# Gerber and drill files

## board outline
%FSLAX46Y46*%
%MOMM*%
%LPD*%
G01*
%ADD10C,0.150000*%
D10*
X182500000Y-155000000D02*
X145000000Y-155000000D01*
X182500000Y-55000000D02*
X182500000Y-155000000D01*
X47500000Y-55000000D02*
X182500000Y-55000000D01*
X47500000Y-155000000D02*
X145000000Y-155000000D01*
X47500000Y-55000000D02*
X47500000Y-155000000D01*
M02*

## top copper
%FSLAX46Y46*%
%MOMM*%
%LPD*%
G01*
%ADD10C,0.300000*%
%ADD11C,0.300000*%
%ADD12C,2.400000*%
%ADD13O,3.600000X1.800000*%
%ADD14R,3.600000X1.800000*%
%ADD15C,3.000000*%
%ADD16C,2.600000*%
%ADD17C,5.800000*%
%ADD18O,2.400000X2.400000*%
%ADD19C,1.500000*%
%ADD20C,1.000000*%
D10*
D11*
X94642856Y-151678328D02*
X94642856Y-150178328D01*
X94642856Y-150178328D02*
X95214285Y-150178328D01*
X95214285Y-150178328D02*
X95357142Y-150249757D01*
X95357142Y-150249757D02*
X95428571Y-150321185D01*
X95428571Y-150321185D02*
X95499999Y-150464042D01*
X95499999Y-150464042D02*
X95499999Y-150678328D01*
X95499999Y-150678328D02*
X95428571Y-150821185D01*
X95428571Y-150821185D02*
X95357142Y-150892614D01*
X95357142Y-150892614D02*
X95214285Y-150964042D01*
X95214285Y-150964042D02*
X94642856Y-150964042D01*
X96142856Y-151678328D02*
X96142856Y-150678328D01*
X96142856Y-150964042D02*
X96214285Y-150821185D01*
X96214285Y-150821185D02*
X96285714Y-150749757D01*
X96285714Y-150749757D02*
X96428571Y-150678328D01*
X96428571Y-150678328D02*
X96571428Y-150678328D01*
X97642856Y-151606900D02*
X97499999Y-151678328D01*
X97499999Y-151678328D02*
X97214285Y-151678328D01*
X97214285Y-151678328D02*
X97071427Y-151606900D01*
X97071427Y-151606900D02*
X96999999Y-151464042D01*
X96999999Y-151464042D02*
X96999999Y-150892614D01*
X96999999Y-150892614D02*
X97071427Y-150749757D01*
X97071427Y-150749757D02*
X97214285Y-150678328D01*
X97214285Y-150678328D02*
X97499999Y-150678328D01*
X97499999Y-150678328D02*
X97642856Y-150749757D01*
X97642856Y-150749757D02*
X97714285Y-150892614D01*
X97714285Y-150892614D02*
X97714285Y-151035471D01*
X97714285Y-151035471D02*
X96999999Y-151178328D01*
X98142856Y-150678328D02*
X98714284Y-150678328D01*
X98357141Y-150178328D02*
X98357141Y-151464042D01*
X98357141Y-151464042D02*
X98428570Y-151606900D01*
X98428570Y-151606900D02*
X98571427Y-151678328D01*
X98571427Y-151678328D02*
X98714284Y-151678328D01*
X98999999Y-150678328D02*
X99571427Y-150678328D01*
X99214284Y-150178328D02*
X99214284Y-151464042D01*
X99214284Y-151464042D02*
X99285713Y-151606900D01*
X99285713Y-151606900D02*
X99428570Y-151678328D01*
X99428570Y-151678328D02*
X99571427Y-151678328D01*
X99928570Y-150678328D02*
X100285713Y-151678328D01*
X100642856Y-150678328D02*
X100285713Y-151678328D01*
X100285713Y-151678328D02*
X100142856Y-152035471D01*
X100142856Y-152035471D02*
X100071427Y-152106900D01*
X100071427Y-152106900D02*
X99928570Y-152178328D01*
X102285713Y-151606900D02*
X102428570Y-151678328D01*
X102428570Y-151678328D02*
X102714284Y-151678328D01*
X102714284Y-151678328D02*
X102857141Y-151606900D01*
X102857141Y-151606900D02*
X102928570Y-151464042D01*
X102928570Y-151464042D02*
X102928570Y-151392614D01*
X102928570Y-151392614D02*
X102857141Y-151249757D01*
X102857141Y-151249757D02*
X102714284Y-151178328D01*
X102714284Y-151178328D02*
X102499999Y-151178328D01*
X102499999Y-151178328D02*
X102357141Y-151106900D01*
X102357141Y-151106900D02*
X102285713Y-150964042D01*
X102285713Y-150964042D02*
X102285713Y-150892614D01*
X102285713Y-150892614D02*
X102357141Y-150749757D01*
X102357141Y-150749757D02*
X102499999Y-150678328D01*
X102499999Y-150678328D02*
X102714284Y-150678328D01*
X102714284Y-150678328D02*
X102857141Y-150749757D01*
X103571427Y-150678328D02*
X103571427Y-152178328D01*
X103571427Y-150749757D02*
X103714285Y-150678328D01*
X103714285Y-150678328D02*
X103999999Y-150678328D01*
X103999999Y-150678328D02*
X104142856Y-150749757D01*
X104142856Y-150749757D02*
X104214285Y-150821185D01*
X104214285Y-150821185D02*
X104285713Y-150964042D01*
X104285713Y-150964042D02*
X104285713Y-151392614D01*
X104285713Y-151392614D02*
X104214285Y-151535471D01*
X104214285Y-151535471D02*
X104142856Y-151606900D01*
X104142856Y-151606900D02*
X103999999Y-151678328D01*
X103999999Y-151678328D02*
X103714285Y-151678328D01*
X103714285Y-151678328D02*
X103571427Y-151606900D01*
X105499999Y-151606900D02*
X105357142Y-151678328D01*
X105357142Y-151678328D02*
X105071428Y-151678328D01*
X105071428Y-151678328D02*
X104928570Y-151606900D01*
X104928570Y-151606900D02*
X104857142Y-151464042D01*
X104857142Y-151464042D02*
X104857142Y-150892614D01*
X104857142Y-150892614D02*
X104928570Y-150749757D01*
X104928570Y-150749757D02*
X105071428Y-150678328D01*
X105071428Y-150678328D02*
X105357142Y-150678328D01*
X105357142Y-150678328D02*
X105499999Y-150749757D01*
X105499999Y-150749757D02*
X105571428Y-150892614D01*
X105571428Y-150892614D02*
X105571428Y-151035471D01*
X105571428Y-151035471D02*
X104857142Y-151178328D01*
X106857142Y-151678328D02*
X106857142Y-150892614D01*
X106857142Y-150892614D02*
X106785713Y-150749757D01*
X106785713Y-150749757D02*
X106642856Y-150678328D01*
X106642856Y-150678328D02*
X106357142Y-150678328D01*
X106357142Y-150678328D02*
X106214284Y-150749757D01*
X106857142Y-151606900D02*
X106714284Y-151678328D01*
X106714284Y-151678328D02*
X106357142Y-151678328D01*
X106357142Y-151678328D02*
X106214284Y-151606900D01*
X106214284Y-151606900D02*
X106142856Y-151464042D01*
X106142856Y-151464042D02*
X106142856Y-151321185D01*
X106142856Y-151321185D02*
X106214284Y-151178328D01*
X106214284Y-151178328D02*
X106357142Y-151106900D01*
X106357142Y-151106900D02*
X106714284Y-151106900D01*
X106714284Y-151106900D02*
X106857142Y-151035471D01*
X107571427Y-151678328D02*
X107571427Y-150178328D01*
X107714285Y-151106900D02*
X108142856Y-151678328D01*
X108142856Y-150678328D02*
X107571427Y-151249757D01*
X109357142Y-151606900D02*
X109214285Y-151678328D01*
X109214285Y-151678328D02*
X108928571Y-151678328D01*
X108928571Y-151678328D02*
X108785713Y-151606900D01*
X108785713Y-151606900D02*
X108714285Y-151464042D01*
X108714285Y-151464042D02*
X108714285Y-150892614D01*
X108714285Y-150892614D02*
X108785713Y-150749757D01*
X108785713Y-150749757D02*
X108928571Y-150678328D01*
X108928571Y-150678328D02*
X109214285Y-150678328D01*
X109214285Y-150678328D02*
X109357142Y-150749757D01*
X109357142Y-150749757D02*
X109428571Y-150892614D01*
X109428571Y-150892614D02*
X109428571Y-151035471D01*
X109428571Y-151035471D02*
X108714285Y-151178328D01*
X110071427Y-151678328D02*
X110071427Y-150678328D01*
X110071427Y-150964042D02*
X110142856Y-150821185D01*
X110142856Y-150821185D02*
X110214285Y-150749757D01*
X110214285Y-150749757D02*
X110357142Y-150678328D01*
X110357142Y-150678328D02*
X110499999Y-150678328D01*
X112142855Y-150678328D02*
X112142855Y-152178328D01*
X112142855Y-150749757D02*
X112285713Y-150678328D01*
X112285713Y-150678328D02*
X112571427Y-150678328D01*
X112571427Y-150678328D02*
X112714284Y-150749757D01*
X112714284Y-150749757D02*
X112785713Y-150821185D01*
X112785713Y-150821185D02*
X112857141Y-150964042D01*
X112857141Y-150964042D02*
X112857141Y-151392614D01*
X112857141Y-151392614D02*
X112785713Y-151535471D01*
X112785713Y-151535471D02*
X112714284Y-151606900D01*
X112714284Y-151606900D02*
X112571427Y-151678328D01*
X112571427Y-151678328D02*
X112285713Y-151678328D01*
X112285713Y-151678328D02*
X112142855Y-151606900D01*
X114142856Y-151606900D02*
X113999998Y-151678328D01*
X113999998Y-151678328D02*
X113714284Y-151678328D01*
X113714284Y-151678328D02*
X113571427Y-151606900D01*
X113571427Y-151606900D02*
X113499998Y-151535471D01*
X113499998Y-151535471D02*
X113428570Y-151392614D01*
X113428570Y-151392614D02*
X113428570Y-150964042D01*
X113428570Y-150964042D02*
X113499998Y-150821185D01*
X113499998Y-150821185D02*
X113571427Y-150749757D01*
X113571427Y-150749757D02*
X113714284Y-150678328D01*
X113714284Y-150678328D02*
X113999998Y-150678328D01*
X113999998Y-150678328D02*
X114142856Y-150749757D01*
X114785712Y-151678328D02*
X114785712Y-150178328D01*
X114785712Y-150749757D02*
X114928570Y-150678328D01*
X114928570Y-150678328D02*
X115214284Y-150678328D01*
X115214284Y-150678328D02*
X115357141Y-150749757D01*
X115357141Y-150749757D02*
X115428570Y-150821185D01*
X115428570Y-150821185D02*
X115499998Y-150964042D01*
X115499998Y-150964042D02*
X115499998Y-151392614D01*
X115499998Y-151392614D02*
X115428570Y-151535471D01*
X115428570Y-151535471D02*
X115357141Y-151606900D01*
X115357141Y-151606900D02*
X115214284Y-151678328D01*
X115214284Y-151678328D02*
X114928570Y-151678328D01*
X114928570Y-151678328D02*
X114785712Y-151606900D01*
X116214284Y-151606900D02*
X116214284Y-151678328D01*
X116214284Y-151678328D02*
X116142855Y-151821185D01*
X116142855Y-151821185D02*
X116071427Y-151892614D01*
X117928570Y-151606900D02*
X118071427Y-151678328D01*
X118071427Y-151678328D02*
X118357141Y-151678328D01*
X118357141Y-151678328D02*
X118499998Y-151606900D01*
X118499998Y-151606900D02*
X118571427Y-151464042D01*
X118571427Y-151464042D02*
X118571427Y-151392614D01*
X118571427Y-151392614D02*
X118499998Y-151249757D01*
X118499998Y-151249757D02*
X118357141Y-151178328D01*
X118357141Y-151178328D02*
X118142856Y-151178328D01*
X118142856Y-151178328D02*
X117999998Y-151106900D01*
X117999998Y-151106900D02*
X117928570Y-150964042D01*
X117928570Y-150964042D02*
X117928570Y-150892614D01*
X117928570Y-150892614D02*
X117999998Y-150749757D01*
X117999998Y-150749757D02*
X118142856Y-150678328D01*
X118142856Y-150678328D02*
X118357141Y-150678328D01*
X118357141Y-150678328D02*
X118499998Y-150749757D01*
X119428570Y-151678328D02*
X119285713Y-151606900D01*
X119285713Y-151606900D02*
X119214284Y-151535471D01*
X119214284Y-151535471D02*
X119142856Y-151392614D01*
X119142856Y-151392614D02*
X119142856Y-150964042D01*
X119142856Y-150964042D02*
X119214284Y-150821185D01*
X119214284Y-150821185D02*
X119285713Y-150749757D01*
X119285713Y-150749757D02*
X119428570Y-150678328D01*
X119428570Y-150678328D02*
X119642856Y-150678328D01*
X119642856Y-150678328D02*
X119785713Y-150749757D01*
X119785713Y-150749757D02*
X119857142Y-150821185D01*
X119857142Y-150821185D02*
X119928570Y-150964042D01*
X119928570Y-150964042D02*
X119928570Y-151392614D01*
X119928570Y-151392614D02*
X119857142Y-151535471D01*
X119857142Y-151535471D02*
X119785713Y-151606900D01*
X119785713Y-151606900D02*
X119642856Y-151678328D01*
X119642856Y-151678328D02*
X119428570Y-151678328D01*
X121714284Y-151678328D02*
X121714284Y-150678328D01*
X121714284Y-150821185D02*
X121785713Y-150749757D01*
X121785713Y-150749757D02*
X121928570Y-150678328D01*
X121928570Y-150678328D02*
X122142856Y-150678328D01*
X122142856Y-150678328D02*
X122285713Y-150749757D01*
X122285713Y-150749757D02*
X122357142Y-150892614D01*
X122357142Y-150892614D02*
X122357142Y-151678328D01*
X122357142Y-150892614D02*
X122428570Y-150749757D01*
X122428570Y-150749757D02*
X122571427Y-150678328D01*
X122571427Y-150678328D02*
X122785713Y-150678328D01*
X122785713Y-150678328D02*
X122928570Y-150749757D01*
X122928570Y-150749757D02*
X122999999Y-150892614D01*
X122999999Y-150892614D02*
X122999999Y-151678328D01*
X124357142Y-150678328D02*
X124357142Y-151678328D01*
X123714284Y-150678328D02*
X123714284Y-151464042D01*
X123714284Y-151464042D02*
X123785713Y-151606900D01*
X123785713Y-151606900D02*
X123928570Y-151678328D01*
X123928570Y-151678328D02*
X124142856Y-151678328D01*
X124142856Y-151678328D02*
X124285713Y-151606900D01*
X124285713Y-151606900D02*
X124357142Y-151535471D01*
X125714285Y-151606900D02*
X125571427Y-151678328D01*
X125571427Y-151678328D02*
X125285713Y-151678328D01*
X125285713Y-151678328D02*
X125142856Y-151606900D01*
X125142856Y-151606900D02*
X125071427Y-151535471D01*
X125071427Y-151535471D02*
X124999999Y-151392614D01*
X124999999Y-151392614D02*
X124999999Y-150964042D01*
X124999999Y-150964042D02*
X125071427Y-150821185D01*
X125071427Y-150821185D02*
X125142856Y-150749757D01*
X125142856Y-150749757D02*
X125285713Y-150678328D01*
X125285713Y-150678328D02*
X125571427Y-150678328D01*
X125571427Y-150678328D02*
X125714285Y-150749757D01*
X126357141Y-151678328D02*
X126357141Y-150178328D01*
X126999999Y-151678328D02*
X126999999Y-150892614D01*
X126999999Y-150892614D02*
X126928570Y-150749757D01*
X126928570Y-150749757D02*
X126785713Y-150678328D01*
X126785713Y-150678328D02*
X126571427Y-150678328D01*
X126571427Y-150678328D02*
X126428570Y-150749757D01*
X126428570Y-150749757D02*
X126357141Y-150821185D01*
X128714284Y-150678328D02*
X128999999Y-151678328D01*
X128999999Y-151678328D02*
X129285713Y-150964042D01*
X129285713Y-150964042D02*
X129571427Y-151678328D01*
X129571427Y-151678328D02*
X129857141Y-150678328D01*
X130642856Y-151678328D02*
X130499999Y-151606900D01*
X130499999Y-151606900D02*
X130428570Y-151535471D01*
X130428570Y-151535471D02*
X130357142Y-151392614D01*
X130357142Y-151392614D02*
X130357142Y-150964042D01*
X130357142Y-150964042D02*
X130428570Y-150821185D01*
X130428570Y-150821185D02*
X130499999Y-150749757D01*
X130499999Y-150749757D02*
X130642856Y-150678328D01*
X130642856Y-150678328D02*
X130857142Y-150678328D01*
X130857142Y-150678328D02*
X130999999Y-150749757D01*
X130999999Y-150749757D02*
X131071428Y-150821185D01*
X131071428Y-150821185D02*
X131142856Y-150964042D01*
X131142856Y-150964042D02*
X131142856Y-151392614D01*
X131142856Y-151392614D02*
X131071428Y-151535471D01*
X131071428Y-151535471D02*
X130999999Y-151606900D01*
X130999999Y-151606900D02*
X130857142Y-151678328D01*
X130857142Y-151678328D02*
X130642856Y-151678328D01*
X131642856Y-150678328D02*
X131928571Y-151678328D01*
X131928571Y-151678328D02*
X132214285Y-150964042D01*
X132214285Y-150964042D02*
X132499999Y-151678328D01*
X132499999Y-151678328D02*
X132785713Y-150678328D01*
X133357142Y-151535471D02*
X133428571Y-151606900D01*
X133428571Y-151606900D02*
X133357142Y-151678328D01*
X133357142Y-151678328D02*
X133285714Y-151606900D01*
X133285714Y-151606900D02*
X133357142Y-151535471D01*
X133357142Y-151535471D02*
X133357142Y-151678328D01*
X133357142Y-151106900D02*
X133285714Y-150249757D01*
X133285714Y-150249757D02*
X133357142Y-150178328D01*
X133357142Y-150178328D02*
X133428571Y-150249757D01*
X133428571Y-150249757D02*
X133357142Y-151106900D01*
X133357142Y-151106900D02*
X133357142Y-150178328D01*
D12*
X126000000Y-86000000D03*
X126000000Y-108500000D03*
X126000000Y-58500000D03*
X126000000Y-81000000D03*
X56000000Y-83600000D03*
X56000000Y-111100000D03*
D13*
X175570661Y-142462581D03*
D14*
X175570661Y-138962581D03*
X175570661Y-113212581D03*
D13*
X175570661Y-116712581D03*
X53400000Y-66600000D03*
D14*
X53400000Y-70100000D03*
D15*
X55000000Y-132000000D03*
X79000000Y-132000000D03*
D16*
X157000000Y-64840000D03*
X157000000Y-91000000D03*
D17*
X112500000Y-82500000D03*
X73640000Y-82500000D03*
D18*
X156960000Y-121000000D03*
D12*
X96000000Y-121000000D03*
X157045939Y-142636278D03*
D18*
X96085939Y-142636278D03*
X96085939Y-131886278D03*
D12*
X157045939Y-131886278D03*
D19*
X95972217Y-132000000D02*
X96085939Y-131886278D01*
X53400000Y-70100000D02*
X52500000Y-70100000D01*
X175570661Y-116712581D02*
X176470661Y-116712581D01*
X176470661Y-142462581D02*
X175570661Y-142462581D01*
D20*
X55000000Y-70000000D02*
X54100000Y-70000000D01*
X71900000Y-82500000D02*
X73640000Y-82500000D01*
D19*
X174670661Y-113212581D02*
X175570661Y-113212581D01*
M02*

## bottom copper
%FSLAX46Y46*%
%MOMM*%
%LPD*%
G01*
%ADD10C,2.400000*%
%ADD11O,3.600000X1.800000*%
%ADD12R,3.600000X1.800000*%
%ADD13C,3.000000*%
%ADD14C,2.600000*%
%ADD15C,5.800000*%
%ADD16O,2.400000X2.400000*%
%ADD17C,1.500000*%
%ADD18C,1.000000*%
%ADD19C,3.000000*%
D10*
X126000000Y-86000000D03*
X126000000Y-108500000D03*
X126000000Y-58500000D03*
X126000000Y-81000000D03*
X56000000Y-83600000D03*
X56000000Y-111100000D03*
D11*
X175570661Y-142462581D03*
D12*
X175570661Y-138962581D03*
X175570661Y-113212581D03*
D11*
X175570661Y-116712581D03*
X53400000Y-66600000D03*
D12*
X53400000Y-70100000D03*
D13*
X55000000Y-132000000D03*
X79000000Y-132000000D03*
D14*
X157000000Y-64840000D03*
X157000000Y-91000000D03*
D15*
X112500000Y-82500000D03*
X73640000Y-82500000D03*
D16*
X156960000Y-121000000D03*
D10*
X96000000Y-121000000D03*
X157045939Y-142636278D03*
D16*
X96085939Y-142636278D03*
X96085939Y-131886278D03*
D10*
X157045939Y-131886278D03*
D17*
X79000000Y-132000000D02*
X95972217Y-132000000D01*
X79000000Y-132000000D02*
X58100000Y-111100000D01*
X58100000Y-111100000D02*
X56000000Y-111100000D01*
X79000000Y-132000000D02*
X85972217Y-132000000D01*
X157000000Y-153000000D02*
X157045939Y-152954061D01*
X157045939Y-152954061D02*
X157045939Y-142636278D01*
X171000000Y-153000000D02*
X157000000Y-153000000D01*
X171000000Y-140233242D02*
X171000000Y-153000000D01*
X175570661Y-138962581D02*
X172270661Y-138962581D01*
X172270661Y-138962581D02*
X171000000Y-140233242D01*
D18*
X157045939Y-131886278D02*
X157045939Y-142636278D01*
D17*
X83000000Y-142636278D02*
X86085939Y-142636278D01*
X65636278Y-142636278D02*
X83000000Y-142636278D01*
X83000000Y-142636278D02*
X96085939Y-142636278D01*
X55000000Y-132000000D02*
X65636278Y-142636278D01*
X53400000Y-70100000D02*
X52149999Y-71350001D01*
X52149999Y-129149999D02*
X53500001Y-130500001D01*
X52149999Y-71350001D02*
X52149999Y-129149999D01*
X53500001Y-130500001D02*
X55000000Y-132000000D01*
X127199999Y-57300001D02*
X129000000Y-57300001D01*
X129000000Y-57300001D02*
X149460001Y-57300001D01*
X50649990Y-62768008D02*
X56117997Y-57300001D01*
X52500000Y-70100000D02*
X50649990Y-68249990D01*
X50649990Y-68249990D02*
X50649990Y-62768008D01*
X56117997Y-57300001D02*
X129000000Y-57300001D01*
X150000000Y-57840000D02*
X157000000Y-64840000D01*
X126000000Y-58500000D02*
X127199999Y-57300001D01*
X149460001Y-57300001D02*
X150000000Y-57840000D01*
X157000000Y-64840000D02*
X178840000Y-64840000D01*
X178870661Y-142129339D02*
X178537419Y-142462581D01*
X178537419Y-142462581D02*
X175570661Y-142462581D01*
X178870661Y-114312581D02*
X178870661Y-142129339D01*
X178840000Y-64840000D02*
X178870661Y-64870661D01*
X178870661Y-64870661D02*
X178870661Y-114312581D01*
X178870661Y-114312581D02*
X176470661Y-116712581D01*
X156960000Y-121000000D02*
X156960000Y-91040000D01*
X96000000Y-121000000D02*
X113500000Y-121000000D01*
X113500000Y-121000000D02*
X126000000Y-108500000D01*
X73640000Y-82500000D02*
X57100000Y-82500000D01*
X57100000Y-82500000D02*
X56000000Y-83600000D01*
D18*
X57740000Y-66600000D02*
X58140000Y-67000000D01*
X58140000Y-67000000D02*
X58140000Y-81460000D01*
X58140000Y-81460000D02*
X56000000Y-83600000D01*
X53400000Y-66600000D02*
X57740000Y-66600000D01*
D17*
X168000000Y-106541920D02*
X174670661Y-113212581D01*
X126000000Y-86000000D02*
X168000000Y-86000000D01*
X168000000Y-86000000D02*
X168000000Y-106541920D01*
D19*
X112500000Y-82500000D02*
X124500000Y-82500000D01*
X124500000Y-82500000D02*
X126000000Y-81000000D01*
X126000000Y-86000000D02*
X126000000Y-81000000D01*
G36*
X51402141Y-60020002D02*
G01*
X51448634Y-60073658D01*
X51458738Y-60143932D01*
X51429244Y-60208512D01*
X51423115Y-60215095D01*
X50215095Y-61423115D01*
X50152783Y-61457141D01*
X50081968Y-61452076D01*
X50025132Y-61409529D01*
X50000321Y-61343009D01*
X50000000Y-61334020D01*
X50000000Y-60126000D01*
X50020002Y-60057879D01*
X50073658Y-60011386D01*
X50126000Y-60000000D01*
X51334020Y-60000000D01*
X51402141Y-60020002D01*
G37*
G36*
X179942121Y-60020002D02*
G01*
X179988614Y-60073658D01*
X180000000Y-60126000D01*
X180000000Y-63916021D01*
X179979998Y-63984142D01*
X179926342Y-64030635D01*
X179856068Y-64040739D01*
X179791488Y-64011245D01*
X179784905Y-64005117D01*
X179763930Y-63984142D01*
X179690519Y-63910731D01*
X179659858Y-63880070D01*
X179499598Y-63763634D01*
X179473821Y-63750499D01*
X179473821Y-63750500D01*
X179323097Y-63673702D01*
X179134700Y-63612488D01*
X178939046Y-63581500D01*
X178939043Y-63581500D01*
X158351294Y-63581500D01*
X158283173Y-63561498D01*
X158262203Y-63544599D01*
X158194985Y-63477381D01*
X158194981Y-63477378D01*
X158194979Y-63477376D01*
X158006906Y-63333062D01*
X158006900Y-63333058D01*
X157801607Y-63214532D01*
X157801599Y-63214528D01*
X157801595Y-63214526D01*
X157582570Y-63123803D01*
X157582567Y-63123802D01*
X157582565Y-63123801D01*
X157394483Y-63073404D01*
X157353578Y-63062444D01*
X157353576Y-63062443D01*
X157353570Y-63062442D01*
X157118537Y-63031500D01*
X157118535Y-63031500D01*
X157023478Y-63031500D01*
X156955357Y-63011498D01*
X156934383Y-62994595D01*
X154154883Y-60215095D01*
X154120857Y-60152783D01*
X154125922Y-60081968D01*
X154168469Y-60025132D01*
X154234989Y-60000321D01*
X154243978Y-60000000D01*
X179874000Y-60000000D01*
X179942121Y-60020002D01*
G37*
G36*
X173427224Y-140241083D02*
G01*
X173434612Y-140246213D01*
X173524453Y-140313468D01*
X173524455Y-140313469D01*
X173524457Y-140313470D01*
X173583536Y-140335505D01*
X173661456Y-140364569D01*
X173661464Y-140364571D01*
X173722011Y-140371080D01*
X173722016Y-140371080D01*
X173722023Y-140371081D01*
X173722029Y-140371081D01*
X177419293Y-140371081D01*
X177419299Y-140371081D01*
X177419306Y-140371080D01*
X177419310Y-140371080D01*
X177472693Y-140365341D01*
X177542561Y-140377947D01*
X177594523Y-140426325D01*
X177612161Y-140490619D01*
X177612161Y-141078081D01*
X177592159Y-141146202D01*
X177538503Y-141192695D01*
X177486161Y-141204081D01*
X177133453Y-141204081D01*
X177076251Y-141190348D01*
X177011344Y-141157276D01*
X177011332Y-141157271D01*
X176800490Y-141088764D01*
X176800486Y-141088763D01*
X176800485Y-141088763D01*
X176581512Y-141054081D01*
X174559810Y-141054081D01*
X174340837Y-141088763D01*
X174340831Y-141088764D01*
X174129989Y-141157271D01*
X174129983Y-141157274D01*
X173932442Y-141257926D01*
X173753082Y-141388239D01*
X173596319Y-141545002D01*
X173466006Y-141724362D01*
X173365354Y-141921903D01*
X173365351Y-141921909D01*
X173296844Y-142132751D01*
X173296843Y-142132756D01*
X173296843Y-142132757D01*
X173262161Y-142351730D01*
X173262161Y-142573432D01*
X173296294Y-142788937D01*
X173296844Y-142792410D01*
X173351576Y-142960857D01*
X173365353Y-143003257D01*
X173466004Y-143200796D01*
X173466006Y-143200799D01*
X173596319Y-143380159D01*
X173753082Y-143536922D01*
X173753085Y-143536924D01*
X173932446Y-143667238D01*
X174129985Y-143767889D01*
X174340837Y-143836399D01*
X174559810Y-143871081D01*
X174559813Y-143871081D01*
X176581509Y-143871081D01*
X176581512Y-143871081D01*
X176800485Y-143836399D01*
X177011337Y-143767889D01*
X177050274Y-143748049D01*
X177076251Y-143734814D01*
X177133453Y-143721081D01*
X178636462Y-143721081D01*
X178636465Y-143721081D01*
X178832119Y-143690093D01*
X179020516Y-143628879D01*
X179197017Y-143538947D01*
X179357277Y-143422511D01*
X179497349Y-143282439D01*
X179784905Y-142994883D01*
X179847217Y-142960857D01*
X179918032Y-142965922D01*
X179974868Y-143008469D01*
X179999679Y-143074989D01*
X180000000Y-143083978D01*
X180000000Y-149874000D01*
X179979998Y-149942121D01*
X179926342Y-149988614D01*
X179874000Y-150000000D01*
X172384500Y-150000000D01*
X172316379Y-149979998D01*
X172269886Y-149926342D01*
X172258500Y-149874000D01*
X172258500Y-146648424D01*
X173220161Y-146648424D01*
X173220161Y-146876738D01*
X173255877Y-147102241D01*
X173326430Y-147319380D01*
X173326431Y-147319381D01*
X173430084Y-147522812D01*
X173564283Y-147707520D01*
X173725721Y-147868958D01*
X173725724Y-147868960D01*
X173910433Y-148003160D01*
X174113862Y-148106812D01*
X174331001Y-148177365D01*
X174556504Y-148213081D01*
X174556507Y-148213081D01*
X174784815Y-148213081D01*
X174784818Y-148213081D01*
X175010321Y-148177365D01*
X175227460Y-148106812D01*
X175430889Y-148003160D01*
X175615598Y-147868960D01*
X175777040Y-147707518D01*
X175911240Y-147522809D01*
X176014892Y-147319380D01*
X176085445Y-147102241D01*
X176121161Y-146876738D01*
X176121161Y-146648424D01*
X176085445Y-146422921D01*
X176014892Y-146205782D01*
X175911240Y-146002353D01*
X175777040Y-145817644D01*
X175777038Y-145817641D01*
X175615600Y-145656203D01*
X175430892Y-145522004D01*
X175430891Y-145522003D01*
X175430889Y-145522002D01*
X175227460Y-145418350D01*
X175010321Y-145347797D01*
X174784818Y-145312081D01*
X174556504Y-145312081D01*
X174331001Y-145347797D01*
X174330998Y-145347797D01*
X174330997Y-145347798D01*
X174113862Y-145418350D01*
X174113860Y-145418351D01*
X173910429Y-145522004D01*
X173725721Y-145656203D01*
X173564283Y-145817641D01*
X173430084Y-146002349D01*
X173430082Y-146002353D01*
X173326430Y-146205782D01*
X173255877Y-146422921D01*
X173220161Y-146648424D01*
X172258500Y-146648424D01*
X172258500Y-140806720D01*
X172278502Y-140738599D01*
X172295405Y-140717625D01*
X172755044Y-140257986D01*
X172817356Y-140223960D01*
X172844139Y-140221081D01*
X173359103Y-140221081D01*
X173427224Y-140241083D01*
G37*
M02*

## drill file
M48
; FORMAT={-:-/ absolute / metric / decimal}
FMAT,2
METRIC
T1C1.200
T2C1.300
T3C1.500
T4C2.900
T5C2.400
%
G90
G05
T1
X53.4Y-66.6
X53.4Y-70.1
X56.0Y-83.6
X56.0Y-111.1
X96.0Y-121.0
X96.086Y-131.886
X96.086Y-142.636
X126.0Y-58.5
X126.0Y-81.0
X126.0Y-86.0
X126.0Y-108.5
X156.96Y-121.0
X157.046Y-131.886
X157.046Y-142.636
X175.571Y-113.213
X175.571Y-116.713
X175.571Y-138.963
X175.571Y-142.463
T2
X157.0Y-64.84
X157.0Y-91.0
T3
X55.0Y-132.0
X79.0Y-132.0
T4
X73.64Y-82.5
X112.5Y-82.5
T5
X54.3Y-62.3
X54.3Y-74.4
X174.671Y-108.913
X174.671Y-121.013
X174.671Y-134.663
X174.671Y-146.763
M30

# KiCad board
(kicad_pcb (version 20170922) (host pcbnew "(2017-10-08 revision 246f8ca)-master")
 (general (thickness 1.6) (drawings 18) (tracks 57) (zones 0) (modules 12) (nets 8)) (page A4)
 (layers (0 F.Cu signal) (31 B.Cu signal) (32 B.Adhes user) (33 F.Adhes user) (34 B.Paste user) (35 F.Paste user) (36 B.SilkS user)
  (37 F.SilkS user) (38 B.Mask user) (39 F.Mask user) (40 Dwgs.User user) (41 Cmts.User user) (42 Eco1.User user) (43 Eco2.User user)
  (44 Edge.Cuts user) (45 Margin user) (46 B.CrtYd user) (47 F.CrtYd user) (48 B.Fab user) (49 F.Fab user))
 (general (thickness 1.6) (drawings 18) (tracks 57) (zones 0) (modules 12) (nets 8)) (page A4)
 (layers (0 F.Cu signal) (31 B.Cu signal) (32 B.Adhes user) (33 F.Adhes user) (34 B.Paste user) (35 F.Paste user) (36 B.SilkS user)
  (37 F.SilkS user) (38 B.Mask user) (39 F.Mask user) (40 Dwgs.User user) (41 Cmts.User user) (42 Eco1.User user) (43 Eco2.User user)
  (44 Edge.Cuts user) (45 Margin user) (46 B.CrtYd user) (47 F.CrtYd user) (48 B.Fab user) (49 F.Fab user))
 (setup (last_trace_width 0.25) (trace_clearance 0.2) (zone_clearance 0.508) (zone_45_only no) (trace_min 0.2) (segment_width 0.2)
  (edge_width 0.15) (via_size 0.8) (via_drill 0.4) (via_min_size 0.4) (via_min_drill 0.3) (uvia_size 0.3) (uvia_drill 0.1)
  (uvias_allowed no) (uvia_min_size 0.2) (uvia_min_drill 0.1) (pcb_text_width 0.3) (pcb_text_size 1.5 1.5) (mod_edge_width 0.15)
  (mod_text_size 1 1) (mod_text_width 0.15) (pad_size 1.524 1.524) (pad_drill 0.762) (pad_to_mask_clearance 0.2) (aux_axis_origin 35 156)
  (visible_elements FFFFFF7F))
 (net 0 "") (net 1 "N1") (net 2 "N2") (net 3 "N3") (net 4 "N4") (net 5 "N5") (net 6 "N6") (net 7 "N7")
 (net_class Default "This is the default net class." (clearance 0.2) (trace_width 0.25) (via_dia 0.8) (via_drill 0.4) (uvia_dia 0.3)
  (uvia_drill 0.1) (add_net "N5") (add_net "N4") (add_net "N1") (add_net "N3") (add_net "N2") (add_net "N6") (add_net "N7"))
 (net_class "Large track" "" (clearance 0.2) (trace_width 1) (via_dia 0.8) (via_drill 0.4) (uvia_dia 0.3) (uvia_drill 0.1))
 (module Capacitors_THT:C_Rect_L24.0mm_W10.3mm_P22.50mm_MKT (layer F.Cu) (at 126 86 270)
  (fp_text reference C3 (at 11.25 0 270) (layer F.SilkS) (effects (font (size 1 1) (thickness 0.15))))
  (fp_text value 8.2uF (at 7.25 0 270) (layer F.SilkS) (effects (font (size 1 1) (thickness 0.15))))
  (pad 1 thru_hole circle (at 0 0 270) (size 2.4 2.4) (drill 1.2) (layers *.Cu *.Mask) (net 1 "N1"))
  (pad 2 thru_hole circle (at 22.5 0 270) (size 2.4 2.4) (drill 1.2) (layers *.Cu *.Mask) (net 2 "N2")))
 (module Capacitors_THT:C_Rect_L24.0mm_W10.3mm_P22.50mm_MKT (layer F.Cu) (at 126 81 90)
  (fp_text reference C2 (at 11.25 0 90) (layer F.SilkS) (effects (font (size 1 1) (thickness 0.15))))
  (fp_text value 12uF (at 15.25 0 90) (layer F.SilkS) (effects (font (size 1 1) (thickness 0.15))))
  (pad 2 thru_hole circle (at 22.5 0 90) (size 2.4 2.4) (drill 1.2) (layers *.Cu *.Mask) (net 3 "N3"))
  (pad 1 thru_hole circle (at 0 0 90) (size 2.4 2.4) (drill 1.2) (layers *.Cu *.Mask) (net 1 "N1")))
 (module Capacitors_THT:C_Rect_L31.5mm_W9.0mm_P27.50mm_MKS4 (layer F.Cu) (at 56 111.1 90)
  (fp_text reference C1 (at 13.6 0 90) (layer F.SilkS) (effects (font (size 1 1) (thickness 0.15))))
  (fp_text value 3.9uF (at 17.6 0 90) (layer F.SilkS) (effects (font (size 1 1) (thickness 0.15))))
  (pad 2 thru_hole circle (at 27.5 0 90) (size 2.4 2.4) (drill 1.2) (layers *.Cu *.Mask) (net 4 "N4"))
  (pad 1 thru_hole circle (at 0 0 90) (size 2.4 2.4) (drill 1.2) (layers *.Cu *.Mask) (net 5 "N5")))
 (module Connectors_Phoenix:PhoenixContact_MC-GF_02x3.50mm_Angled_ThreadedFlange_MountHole (layer F.Cu) (at 175.570661 138.962581 270)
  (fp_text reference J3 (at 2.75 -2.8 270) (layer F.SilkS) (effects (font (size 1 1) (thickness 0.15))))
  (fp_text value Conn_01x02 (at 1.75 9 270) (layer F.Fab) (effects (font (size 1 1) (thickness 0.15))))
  (pad "" np_thru_hole circle (at 7.8 0.9 270) (size 2.4 2.4) (drill 2.4) (layers *.Cu *.Mask))
  (pad "" np_thru_hole circle (at -4.3 0.9 270) (size 2.4 2.4) (drill 2.4) (layers *.Cu *.Mask))
  (pad 2 thru_hole oval (at 3.5 0 270) (size 1.8 3.6) (drill 1.2) (layers *.Cu *.Mask) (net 3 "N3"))
  (pad 1 thru_hole rect (at 0 0 270) (size 1.8 3.6) (drill 1.2) (layers *.Cu *.Mask) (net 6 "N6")))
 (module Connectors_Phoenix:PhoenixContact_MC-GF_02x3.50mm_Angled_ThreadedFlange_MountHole (layer F.Cu) (at 175.570661 113.212581 270)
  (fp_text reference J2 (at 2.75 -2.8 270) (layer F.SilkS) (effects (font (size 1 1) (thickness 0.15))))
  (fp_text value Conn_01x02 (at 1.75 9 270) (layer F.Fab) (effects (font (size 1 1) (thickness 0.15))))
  (pad 1 thru_hole rect (at 0 0 270) (size 1.8 3.6) (drill 1.2) (layers *.Cu *.Mask) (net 1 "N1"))
  (pad 2 thru_hole oval (at 3.5 0 270) (size 1.8 3.6) (drill 1.2) (layers *.Cu *.Mask) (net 3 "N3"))
  (pad "" np_thru_hole circle (at -4.3 0.9 270) (size 2.4 2.4) (drill 2.4) (layers *.Cu *.Mask))
  (pad "" np_thru_hole circle (at 7.8 0.9 270) (size 2.4 2.4) (drill 2.4) (layers *.Cu *.Mask)))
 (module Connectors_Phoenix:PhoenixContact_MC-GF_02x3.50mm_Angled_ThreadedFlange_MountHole (layer F.Cu) (at 53.4 70.1 90)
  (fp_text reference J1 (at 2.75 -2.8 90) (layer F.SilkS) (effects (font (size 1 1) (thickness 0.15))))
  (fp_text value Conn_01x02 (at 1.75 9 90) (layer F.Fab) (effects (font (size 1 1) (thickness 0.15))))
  (pad "" np_thru_hole circle (at 7.8 0.9 90) (size 2.4 2.4) (drill 2.4) (layers *.Cu *.Mask))
  (pad "" np_thru_hole circle (at -4.3 0.9 90) (size 2.4 2.4) (drill 2.4) (layers *.Cu *.Mask))
  (pad 2 thru_hole oval (at 3.5 0 90) (size 1.8 3.6) (drill 1.2) (layers *.Cu *.Mask) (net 4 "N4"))
  (pad 1 thru_hole rect (at 0 0 90) (size 1.8 3.6) (drill 1.2) (layers *.Cu *.Mask) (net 3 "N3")))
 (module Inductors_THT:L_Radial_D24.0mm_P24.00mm (layer F.Cu) (at 79 132 180)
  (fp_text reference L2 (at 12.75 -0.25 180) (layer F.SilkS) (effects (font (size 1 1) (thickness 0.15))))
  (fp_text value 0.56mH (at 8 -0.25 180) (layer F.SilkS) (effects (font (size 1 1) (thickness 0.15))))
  (pad 2 thru_hole circle (at 24 0 180) (size 3 3) (drill 1.5) (layers *.Cu *.Mask) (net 3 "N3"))
  (pad 1 thru_hole circle (at 0 0 180) (size 3 3) (drill 1.5) (layers *.Cu *.Mask) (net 5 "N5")))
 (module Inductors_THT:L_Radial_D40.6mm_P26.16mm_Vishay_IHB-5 (layer F.Cu) (at 157 91 90)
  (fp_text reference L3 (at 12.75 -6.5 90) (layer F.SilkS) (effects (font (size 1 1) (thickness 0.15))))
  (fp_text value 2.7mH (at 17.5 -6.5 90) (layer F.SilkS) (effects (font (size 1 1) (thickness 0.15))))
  (pad 2 thru_hole circle (at 26.16 0 90) (size 2.6 2.6) (drill 1.3) (layers *.Cu *.Mask) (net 3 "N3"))
  (pad 1 thru_hole circle (at 0 0 90) (size 2.6 2.6) (drill 1.3) (layers *.Cu *.Mask) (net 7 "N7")))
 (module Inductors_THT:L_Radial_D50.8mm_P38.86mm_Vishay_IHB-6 (layer F.Cu) (at 112.5 82.5 180)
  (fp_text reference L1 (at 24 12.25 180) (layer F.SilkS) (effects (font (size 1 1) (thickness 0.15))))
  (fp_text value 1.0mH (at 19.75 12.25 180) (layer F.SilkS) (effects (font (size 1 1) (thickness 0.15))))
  (pad 1 thru_hole circle (at 0 0 180) (size 5.8 5.8) (drill 2.9) (layers *.Cu *.Mask) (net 1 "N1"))
  (pad 2 thru_hole circle (at 38.86 0 180) (size 5.8 5.8) (drill 2.9) (layers *.Cu *.Mask) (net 4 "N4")))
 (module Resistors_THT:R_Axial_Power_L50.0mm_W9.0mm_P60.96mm (layer F.Cu) (at 96 121)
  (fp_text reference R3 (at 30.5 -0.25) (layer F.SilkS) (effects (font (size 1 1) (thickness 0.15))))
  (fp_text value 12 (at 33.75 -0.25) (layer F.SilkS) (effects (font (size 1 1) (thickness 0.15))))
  (pad 2 thru_hole oval (at 60.96 0) (size 2.4 2.4) (drill 1.2) (layers *.Cu *.Mask) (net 7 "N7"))
  (pad 1 thru_hole circle (at 0 0) (size 2.4 2.4) (drill 1.2) (layers *.Cu *.Mask) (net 2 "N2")))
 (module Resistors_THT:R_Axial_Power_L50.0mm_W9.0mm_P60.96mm (layer F.Cu) (at 157.045939 142.636278 180)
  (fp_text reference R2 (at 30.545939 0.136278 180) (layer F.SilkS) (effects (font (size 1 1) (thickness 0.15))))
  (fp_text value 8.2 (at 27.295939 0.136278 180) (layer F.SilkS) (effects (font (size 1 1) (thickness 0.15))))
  (pad 1 thru_hole circle (at 0 0 180) (size 2.4 2.4) (drill 1.2) (layers *.Cu *.Mask) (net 6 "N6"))
  (pad 2 thru_hole oval (at 60.96 0 180) (size 2.4 2.4) (drill 1.2) (layers *.Cu *.Mask) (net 3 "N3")))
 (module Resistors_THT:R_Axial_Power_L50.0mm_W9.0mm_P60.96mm (layer F.Cu) (at 157.045939 131.886278 180)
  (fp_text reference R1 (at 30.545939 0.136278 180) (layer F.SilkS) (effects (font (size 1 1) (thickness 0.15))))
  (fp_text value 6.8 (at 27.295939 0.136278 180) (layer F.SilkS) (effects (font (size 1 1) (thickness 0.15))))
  (pad 2 thru_hole oval (at 60.96 0 180) (size 2.4 2.4) (drill 1.2) (layers *.Cu *.Mask) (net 5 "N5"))
  (pad 1 thru_hole circle (at 0 0 180) (size 2.4 2.4) (drill 1.2) (layers *.Cu *.Mask) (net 6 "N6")))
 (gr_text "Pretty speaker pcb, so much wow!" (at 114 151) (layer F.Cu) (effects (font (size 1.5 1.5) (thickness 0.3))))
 (gr_line (start 182.5 155) (end 145 155) (layer Edge.Cuts) (width 0.15))
 (gr_line (start 182.5 55) (end 182.5 155) (layer Edge.Cuts) (width 0.15))
 (gr_line (start 47.5 55) (end 182.5 55) (layer Edge.Cuts) (width 0.15))
 (gr_line (start 47.5 155) (end 145 155) (layer Edge.Cuts) (width 0.15))
 (gr_line (start 47.5 55) (end 47.5 155) (layer Edge.Cuts) (width 0.15))
 (segment (start 79 132) (end 95.972217 132) (width 1.5) (layer B.Cu) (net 5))
 (segment (start 95.972217 132) (end 96.085939 131.886278) (width 1.5) (layer F.Cu) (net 5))
 (segment (start 79 132) (end 58.1 111.1) (width 1.5) (layer B.Cu) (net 5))
 (segment (start 58.1 111.1) (end 56 111.1) (width 1.5) (layer B.Cu) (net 5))
 (segment (start 79 132) (end 85.972217 132) (width 1.5) (layer B.Cu) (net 5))
 (segment (start 157 153) (end 157.045939 152.954061) (width 1.5) (layer B.Cu) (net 6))
 (segment (start 157.045939 152.954061) (end 157.045939 142.636278) (width 1.5) (layer B.Cu) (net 6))
 (segment (start 171 153) (end 157 153) (width 1.5) (layer B.Cu) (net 6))
 (segment (start 171 140.233242) (end 171 153) (width 1.5) (layer B.Cu) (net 6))
 (segment (start 175.570661 138.962581) (end 172.270661 138.962581) (width 1.5) (layer B.Cu) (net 6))
 (segment (start 172.270661 138.962581) (end 171 140.233242) (width 1.5) (layer B.Cu) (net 6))
 (segment (start 157.045939 131.886278) (end 157.045939 142.636278) (width 1) (layer B.Cu) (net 6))
 (segment (start 83 142.636278) (end 86.085939 142.636278) (width 1.5) (layer B.Cu) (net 3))
 (segment (start 65.636278 142.636278) (end 83 142.636278) (width 1.5) (layer B.Cu) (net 3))
 (segment (start 83 142.636278) (end 96.085939 142.636278) (width 1.5) (layer B.Cu) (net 3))
 (segment (start 55 132) (end 65.636278 142.636278) (width 1.5) (layer B.Cu) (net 3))
 (segment (start 53.4 70.1) (end 52.149999 71.350001) (width 1.5) (layer B.Cu) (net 3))
 (segment (start 52.149999 129.149999) (end 53.500001 130.500001) (width 1.5) (layer B.Cu) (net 3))
 (segment (start 52.149999 71.350001) (end 52.149999 129.149999) (width 1.5) (layer B.Cu) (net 3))
 (segment (start 53.500001 130.500001) (end 55 132) (width 1.5) (layer B.Cu) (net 3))
 (segment (start 127.199999 57.300001) (end 129 57.300001) (width 1.5) (layer B.Cu) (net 3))
 (segment (start 129 57.300001) (end 149.460001 57.300001) (width 1.5) (layer B.Cu) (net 3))
 (segment (start 50.64999 62.768008) (end 56.117997 57.300001) (width 1.5) (layer B.Cu) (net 3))
 (segment (start 53.4 70.1) (end 52.5 70.1) (width 1.5) (layer F.Cu) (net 3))
 (segment (start 52.5 70.1) (end 50.64999 68.24999) (width 1.5) (layer B.Cu) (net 3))
 (segment (start 50.64999 68.24999) (end 50.64999 62.768008) (width 1.5) (layer B.Cu) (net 3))
 (segment (start 56.117997 57.300001) (end 129 57.300001) (width 1.5) (layer B.Cu) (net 3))
 (segment (start 150 57.84) (end 157 64.84) (width 1.5) (layer B.Cu) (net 3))
 (segment (start 126 58.5) (end 127.199999 57.300001) (width 1.5) (layer B.Cu) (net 3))
 (segment (start 149.460001 57.300001) (end 150 57.84) (width 1.5) (layer B.Cu) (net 3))
 (segment (start 157 64.84) (end 178.84 64.84) (width 1.5) (layer B.Cu) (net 3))
 (segment (start 178.870661 142.129339) (end 178.537419 142.462581) (width 1.5) (layer B.Cu) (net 3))
 (segment (start 178.537419 142.462581) (end 175.570661 142.462581) (width 1.5) (layer B.Cu) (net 3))
 (segment (start 178.870661 114.312581) (end 178.870661 142.129339) (width 1.5) (layer B.Cu) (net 3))
 (segment (start 175.570661 116.712581) (end 176.470661 116.712581) (width 1.5) (layer F.Cu) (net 3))
 (segment (start 176.470661 142.462581) (end 175.570661 142.462581) (width 1.5) (layer F.Cu) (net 3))
 (segment (start 178.84 64.84) (end 178.870661 64.870661) (width 1.5) (layer B.Cu) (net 3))
 (segment (start 178.870661 64.870661) (end 178.870661 114.312581) (width 1.5) (layer B.Cu) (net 3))
 (segment (start 178.870661 114.312581) (end 176.470661 116.712581) (width 1.5) (layer B.Cu) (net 3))
 (segment (start 55 70) (end 54.1 70) (width 1) (layer F.Cu) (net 3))
 (segment (start 156.96 121) (end 156.96 91.04) (width 1.5) (layer B.Cu) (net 7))
 (segment (start 96 121) (end 113.5 121) (width 1.5) (layer B.Cu) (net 2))
 (segment (start 113.5 121) (end 126 108.5) (width 1.5) (layer B.Cu) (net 2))
 (segment (start 73.64 82.5) (end 57.1 82.5) (width 1.5) (layer B.Cu) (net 4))
 (segment (start 57.1 82.5) (end 56 83.6) (width 1.5) (layer B.Cu) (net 4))
 (segment (start 57.74 66.6) (end 58.14 67) (width 1) (layer B.Cu) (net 4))
 (segment (start 58.14 67) (end 58.14 81.46) (width 1) (layer B.Cu) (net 4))
 (segment (start 58.14 81.46) (end 56 83.6) (width 1) (layer B.Cu) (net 4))
 (segment (start 53.4 66.6) (end 57.74 66.6) (width 1) (layer B.Cu) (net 4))
 (segment (start 71.9 82.5) (end 73.64 82.5) (width 1) (layer F.Cu) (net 4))
 (segment (start 168 106.54192) (end 174.670661 113.212581) (width 1.5) (layer B.Cu) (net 1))
 (segment (start 126 86) (end 168 86) (width 1.5) (layer B.Cu) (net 1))
 (segment (start 168 86) (end 168 106.54192) (width 1.5) (layer B.Cu) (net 1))
 (segment (start 174.670661 113.212581) (end 175.570661 113.212581) (width 1.5) (layer F.Cu) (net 1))
 (segment (start 112.5 82.5) (end 124.5 82.5) (width 3) (layer B.Cu) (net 1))
 (segment (start 124.5 82.5) (end 126 81) (width 3) (layer B.Cu) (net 1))
 (segment (start 126 86) (end 126 81) (width 3) (layer B.Cu) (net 1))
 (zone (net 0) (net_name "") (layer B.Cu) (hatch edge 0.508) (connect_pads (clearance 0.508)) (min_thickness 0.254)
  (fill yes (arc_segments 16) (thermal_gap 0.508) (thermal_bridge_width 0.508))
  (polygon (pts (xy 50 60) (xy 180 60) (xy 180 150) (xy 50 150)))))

